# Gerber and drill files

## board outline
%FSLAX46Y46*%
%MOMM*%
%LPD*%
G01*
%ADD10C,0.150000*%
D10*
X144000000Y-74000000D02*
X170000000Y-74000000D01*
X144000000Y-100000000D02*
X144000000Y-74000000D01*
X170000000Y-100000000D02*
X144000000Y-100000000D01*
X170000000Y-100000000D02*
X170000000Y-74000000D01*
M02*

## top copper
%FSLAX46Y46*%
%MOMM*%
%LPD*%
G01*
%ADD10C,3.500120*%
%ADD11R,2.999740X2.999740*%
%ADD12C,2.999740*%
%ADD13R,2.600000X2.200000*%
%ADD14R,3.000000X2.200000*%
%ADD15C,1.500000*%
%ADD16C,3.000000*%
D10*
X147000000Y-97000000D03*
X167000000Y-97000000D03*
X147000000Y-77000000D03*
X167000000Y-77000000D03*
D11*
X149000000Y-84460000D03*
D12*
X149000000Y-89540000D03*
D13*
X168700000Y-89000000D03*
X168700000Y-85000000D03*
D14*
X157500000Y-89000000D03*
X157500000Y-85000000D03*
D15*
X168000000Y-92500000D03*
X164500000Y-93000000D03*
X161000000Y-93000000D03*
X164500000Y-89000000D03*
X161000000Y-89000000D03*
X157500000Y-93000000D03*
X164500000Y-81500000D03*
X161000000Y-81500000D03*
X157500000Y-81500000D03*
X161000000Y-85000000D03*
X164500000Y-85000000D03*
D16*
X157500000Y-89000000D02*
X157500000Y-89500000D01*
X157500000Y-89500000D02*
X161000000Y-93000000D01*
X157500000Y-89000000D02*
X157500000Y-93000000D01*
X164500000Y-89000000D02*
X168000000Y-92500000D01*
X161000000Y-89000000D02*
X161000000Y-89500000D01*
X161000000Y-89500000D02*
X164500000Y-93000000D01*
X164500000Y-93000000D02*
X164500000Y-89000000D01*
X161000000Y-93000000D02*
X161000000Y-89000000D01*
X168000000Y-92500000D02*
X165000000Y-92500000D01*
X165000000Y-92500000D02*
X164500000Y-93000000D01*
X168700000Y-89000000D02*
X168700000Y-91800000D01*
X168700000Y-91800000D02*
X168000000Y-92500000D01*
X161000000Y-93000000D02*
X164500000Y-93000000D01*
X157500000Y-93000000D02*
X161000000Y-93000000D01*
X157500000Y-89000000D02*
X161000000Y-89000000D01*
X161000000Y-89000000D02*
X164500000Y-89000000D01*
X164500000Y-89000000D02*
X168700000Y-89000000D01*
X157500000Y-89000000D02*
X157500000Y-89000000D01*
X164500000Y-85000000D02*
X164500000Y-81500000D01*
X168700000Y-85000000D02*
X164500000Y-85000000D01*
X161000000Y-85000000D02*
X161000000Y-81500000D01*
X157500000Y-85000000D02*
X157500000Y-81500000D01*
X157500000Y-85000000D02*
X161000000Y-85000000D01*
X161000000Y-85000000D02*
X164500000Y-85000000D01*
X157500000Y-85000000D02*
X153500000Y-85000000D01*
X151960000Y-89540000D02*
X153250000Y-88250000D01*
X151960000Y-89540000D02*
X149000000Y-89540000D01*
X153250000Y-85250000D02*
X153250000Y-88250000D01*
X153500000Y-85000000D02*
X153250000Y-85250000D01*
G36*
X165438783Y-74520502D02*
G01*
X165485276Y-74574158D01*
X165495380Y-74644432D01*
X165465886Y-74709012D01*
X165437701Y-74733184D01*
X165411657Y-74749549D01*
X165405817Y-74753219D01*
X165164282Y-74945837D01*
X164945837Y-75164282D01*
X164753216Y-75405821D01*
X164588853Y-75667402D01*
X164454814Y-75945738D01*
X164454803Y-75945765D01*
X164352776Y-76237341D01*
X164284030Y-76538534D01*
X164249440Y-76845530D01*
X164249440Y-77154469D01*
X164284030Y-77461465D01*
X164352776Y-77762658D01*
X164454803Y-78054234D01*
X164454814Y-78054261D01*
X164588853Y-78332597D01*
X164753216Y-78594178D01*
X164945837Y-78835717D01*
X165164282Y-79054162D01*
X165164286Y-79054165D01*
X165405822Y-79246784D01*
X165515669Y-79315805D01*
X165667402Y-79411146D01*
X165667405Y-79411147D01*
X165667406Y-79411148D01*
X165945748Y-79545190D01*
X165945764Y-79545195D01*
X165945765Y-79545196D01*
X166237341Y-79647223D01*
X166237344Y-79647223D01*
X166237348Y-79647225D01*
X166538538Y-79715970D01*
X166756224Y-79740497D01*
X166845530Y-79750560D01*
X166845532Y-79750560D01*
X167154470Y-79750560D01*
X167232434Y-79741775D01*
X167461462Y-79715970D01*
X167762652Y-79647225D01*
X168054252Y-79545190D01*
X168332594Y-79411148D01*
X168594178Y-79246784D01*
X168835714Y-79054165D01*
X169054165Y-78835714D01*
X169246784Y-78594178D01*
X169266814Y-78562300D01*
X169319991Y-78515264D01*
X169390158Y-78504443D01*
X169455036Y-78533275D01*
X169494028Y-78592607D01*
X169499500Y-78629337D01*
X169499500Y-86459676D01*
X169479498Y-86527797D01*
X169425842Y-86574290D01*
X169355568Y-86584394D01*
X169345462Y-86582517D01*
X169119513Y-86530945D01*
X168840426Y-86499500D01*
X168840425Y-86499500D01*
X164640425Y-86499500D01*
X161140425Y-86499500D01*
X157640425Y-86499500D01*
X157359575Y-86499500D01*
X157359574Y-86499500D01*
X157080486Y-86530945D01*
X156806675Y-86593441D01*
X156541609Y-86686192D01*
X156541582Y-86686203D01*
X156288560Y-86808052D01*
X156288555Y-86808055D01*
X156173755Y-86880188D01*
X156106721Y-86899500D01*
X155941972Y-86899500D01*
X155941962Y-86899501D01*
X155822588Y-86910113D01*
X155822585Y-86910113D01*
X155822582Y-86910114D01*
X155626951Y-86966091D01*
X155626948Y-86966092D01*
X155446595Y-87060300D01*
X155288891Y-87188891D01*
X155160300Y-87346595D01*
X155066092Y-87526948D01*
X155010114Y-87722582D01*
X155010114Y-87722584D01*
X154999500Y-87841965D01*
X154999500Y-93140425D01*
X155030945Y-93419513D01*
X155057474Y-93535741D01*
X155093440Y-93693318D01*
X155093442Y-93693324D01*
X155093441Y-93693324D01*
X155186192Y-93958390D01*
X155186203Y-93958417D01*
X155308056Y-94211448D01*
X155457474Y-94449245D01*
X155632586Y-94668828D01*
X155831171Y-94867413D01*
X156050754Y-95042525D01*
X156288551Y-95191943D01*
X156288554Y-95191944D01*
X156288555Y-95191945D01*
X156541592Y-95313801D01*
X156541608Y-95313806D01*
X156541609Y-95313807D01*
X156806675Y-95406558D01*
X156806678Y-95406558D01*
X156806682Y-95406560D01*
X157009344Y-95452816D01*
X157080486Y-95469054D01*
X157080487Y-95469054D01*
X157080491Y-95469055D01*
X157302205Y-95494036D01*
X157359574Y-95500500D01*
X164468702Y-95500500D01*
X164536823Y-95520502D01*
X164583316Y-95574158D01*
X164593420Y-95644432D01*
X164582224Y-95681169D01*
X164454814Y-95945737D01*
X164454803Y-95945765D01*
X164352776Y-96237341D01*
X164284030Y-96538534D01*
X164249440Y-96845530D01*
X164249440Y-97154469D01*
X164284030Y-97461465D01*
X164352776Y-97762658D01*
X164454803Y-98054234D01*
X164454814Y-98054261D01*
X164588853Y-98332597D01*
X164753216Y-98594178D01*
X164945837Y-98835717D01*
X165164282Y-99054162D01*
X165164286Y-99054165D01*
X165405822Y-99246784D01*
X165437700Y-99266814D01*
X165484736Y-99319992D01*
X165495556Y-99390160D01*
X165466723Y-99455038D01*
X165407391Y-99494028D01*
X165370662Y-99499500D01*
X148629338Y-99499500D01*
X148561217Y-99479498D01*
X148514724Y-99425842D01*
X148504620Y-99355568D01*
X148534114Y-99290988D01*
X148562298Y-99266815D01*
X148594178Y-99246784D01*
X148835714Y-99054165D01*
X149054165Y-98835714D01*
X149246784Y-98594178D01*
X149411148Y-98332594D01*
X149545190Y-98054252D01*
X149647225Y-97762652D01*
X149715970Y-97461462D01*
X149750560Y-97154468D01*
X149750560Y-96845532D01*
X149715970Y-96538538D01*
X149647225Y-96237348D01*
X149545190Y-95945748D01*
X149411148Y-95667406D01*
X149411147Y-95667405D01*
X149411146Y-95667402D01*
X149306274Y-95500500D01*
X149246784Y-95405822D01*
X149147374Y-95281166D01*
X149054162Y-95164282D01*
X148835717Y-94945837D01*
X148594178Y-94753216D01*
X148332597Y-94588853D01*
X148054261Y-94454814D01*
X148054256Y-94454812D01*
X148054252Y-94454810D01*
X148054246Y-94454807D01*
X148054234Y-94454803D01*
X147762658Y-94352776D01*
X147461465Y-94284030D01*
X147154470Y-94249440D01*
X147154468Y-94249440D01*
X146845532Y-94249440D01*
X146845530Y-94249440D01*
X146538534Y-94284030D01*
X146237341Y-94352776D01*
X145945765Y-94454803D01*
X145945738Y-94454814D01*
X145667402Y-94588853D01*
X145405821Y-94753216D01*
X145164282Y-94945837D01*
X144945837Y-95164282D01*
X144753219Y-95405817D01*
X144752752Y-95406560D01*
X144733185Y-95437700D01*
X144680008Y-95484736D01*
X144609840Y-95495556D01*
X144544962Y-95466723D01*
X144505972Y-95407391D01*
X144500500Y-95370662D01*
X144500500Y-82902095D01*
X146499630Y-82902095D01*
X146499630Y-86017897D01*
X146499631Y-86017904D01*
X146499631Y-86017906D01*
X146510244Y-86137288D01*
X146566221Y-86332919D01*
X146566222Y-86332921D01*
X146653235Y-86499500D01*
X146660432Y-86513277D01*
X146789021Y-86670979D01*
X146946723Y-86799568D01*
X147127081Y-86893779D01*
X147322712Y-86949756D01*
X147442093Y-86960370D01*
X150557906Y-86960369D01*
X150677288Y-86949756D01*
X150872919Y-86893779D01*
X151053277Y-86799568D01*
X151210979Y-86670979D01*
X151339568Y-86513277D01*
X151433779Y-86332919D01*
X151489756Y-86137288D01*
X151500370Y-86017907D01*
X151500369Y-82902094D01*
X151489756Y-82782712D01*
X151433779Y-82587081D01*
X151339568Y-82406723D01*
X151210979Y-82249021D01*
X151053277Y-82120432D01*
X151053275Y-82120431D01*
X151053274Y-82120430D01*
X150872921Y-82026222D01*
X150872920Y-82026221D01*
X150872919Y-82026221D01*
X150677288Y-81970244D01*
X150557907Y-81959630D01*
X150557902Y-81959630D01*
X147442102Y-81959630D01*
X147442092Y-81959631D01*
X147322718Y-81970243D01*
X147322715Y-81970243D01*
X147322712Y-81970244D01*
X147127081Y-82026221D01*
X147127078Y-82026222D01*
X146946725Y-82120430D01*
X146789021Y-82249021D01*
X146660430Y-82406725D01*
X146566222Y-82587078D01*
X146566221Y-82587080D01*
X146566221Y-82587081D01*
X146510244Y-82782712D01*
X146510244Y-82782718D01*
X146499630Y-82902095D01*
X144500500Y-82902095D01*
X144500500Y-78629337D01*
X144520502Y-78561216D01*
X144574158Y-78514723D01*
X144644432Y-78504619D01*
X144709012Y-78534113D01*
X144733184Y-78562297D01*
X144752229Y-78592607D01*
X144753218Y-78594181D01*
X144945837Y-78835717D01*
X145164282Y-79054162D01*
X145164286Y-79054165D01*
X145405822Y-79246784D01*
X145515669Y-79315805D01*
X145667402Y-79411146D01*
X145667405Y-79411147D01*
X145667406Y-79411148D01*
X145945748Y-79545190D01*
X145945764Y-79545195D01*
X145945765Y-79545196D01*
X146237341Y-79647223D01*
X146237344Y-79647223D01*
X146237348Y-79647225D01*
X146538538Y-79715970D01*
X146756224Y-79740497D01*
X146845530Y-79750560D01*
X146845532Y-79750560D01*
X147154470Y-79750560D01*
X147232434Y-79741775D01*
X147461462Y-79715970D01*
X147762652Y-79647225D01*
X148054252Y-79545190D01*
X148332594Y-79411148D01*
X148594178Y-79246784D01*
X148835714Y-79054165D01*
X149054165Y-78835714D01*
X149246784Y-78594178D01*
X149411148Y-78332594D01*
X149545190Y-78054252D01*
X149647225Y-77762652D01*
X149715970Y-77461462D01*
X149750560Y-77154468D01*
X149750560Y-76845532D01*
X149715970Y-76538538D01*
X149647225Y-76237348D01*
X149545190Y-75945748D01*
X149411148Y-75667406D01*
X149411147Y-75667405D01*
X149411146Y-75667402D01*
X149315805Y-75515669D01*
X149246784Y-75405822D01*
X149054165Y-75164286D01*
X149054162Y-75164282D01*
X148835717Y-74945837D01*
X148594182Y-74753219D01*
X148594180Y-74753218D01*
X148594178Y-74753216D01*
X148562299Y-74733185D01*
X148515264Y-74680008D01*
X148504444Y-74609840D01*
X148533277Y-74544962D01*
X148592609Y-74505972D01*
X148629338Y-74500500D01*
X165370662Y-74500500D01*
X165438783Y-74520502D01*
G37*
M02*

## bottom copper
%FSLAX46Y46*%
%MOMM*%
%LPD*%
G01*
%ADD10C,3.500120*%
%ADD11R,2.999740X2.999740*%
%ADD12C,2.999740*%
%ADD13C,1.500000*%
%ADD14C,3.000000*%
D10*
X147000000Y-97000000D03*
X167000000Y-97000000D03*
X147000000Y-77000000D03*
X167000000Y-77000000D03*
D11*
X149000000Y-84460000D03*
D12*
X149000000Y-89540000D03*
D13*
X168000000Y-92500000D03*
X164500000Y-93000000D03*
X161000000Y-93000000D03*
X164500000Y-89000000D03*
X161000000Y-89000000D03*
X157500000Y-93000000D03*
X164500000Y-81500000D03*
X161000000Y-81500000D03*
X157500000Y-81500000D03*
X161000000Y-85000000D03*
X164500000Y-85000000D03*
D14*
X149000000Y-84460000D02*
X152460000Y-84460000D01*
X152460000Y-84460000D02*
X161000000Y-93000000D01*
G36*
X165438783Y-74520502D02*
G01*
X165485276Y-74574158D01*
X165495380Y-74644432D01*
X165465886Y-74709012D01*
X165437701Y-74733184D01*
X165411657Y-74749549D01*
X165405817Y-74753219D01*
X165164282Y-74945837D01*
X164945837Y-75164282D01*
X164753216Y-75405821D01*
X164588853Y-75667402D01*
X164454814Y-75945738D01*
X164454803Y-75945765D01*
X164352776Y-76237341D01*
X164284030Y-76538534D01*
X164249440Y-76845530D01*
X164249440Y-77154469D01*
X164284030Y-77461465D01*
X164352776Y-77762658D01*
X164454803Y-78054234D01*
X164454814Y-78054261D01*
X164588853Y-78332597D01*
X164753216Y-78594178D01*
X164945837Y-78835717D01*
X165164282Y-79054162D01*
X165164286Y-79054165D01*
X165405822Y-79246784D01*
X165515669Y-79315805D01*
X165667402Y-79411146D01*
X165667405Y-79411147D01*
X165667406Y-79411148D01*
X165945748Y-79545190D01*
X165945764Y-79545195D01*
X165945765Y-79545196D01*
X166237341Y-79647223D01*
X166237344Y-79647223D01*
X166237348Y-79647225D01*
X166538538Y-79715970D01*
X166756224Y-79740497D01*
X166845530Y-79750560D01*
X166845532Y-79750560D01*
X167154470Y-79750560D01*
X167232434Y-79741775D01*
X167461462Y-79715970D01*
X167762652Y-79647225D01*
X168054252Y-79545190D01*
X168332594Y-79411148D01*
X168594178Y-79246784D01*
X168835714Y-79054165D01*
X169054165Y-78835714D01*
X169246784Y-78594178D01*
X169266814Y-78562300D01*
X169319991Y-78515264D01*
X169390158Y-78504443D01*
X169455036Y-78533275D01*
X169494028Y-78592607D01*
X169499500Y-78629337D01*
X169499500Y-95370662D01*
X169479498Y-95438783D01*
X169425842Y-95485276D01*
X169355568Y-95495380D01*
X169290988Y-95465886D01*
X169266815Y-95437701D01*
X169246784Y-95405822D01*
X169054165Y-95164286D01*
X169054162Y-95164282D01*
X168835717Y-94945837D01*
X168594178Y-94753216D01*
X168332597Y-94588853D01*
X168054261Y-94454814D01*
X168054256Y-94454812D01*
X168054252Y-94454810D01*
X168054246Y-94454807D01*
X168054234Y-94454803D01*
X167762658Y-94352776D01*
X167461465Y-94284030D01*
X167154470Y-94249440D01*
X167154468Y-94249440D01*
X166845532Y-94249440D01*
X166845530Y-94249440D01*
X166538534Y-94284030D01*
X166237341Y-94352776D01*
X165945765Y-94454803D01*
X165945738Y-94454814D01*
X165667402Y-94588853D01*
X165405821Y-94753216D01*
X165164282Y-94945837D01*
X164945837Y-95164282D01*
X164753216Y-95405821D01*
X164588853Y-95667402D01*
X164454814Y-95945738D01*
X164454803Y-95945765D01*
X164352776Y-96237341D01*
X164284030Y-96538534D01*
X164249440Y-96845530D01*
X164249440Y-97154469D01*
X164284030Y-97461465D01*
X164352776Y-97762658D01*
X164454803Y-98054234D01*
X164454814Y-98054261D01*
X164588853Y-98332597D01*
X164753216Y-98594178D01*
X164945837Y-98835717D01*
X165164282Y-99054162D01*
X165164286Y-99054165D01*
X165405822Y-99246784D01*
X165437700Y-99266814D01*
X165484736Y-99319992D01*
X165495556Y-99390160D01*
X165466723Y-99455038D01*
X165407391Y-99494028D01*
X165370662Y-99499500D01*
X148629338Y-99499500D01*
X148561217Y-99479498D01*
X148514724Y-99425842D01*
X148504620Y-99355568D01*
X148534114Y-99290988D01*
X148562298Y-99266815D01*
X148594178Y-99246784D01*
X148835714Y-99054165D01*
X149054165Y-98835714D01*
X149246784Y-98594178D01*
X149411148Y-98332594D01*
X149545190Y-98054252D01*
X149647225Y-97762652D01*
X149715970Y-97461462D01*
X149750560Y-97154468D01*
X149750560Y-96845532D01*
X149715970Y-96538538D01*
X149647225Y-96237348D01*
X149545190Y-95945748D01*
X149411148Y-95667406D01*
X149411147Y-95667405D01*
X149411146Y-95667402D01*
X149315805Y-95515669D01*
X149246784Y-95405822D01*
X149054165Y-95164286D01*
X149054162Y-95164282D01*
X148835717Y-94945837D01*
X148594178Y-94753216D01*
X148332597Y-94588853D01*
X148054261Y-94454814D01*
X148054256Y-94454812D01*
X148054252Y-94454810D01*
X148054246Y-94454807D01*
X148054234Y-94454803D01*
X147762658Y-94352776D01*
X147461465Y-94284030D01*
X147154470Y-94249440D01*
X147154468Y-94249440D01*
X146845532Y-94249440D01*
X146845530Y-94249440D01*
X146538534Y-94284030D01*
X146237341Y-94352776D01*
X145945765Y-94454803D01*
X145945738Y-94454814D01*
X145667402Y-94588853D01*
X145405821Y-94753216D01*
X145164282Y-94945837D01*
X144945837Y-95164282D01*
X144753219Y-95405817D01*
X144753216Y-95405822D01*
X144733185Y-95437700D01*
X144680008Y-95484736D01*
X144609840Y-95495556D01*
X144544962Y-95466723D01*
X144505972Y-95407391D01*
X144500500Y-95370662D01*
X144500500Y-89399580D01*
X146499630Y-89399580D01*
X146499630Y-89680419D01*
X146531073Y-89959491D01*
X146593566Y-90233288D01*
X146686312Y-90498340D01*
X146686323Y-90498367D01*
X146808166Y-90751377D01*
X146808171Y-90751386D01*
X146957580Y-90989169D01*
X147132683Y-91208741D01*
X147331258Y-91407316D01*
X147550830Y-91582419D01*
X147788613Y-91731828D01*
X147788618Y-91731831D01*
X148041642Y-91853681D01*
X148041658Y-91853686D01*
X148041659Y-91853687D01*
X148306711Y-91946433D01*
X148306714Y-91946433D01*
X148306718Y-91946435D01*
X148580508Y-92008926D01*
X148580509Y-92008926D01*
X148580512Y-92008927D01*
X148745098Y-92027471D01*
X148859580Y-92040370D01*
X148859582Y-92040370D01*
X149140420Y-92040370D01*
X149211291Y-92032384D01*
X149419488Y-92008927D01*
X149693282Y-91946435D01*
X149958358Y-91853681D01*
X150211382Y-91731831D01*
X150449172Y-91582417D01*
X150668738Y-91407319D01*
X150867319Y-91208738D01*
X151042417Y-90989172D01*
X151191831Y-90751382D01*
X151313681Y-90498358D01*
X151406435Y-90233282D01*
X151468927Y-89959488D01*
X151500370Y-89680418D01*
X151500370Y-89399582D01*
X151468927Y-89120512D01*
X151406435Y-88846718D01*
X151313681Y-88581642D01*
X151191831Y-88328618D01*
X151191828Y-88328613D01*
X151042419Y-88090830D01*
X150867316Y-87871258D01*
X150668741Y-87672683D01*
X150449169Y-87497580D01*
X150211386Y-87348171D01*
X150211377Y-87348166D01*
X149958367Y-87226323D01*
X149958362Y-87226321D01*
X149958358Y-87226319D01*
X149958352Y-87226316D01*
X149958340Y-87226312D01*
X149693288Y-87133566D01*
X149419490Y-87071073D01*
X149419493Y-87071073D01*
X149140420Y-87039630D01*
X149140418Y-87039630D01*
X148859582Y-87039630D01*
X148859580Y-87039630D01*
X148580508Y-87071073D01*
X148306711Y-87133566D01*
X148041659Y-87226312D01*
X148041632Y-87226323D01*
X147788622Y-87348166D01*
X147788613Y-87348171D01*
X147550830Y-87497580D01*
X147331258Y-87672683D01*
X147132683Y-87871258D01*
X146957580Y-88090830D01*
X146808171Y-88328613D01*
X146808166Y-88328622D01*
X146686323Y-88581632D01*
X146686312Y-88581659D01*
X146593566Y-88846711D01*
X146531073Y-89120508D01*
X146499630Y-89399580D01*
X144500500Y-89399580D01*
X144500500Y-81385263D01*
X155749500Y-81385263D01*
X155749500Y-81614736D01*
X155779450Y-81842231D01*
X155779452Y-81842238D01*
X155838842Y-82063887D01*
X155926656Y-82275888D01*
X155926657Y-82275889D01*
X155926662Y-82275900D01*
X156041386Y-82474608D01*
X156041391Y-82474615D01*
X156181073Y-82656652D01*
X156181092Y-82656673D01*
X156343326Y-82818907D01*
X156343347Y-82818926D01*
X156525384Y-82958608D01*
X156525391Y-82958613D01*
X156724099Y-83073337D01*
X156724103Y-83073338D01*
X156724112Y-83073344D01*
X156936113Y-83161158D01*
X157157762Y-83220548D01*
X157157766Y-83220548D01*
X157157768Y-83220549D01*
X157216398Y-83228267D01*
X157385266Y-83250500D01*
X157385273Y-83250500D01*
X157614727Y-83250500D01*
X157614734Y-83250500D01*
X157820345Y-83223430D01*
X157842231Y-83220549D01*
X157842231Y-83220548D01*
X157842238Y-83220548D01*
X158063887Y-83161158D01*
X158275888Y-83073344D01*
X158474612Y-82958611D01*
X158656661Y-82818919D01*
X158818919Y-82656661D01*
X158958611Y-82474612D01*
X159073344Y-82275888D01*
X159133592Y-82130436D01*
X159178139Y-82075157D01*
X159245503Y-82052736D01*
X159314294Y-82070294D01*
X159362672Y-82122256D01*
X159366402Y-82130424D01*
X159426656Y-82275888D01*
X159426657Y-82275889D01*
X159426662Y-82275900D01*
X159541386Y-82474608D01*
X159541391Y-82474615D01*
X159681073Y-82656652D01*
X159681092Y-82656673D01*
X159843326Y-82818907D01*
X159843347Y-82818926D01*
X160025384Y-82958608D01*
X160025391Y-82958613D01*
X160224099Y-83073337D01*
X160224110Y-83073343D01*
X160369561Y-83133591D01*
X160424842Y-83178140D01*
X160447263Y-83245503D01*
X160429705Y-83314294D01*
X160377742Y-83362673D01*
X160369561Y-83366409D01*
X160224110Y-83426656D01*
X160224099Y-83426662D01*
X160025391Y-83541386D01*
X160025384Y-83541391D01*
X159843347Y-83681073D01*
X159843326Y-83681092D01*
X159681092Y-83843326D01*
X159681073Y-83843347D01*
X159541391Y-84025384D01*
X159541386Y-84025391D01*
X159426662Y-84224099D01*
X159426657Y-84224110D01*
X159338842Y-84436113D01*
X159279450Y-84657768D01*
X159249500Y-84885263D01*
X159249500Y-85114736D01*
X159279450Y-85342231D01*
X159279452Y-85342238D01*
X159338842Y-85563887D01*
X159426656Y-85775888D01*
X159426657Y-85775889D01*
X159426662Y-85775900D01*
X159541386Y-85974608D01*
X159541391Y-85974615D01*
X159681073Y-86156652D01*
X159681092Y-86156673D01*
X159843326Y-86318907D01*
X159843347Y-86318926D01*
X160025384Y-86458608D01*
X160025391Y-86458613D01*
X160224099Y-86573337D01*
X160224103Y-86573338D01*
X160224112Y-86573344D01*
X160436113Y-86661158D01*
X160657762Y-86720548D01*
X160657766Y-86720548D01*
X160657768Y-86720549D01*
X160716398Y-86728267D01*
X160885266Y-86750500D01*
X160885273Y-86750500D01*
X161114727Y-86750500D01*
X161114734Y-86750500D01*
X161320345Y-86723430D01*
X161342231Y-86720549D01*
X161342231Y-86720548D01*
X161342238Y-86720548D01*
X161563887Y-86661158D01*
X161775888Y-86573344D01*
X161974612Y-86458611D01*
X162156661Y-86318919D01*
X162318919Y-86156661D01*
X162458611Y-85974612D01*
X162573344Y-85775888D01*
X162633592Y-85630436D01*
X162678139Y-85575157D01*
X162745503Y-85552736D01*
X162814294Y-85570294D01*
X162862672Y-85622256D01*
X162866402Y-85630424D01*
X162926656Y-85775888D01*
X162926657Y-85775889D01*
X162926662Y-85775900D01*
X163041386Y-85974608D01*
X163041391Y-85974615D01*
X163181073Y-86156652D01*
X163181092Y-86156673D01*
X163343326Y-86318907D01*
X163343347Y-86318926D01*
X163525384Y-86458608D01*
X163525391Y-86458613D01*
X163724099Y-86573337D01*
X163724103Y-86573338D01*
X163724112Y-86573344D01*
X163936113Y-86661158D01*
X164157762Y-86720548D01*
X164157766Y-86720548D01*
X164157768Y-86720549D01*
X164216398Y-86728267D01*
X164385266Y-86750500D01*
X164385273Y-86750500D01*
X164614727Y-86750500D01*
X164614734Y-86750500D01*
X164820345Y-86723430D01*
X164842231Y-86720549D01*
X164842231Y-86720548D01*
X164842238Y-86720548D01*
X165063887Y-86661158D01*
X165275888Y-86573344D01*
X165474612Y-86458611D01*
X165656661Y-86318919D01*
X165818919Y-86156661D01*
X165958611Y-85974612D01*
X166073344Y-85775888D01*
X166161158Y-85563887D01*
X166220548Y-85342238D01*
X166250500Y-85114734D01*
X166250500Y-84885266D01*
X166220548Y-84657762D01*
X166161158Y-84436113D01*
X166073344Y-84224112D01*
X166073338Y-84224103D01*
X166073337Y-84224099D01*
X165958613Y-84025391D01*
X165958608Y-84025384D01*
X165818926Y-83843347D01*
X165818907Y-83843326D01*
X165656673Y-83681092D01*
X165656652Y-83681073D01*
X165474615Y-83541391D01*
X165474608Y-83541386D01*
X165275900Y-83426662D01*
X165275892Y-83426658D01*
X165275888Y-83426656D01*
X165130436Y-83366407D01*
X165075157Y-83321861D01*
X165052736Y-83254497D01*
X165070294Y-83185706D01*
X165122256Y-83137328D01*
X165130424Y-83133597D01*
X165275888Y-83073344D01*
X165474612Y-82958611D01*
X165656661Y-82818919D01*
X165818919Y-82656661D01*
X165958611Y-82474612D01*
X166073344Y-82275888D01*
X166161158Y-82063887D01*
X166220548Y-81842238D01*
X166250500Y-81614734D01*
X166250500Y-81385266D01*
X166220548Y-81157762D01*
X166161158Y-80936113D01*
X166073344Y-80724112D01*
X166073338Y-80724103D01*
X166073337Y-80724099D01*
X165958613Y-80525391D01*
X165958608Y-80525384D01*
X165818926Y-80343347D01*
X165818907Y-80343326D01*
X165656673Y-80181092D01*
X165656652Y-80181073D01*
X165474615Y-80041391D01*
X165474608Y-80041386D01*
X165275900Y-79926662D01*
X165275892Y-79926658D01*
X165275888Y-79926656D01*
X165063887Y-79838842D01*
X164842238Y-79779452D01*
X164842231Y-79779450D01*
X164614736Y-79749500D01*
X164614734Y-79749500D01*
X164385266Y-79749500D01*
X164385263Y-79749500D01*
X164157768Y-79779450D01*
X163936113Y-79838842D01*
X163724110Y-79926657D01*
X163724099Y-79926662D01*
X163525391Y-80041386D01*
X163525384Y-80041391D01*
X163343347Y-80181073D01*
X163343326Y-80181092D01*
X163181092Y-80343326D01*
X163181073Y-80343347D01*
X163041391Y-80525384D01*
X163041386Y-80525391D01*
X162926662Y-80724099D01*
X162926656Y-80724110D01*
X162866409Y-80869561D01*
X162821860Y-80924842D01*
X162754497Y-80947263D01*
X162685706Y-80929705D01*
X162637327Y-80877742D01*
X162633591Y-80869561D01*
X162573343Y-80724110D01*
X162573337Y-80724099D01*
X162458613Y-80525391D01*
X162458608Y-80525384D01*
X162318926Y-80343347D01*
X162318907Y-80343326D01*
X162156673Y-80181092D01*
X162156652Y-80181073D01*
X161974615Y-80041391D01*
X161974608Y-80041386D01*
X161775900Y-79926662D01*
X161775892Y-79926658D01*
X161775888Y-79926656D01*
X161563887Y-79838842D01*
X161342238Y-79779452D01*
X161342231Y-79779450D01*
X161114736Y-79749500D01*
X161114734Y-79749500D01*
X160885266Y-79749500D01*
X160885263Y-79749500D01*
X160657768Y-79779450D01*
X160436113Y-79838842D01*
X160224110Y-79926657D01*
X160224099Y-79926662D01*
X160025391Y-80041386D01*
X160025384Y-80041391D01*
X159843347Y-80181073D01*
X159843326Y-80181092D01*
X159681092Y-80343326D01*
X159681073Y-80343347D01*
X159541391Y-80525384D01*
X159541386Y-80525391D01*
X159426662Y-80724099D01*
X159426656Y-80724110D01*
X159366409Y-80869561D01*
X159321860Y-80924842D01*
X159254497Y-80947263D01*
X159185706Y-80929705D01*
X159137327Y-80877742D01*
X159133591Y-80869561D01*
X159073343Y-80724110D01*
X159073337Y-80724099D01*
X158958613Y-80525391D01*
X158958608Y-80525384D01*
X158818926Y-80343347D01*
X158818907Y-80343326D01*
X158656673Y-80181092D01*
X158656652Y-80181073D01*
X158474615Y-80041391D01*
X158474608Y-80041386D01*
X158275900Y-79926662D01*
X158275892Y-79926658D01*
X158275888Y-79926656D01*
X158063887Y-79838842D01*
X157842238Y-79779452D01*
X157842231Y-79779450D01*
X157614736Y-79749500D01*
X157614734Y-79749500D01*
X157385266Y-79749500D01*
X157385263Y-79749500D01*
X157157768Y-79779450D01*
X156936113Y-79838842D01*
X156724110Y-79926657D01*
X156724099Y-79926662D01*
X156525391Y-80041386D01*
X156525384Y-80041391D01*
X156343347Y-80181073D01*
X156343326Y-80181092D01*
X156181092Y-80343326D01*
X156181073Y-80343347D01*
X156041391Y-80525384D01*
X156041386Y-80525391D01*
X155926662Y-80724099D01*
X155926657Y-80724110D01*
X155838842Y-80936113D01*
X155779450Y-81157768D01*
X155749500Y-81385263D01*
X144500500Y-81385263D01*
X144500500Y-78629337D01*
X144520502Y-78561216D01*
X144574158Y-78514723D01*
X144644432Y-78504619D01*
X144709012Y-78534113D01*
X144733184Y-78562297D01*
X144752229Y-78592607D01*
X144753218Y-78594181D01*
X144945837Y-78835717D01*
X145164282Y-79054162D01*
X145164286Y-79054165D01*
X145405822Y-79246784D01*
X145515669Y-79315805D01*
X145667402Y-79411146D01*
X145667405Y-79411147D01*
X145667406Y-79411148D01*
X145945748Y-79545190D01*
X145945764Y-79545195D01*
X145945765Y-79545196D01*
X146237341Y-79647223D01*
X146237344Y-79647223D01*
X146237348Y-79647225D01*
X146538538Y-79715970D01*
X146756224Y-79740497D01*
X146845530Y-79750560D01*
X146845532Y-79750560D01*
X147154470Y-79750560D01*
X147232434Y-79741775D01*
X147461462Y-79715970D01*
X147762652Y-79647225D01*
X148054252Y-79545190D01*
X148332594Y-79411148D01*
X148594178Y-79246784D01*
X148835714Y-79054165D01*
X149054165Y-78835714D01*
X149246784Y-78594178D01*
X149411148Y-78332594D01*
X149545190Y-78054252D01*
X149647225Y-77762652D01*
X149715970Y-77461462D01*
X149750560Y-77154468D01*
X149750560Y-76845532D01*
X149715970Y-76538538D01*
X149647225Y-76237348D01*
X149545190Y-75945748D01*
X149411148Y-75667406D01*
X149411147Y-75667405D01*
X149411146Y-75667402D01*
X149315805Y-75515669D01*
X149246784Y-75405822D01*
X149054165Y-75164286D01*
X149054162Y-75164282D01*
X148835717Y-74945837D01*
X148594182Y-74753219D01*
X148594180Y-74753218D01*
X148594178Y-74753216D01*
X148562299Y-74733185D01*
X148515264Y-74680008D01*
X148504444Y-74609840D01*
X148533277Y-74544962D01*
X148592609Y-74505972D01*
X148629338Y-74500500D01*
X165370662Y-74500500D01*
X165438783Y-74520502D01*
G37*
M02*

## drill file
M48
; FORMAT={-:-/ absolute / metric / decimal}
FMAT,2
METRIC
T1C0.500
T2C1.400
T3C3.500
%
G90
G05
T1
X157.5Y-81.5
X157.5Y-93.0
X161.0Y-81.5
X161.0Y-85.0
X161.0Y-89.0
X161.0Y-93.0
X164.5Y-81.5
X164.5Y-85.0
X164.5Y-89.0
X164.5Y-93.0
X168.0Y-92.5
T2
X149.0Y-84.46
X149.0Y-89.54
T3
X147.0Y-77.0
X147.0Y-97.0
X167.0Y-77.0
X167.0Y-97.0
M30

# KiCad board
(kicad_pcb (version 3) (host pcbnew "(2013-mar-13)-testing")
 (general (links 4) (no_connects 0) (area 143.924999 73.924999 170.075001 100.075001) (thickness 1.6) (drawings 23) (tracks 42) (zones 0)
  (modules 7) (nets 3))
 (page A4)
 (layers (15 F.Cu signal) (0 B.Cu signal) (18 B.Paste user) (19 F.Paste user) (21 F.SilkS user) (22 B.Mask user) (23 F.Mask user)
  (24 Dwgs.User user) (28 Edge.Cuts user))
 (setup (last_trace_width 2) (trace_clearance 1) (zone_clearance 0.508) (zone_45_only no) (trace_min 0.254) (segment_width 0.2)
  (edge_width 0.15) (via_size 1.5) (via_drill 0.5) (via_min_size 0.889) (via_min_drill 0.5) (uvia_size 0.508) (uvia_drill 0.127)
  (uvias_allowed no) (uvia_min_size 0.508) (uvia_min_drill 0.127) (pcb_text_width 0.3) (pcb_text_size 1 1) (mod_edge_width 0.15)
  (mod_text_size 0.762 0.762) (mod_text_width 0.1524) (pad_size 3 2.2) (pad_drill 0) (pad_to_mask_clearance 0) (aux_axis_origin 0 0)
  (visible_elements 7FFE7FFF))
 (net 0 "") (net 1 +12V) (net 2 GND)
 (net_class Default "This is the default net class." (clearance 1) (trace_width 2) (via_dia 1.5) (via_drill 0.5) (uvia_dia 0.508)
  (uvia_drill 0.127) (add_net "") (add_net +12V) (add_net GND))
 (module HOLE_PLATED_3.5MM (layer F.Cu) (at 147 97)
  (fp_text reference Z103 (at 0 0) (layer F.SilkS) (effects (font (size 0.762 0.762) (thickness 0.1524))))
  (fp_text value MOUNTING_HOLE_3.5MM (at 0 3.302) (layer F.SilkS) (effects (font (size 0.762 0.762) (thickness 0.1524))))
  (pad 1 thru_hole circle (at 0 0) (size 3.50012 3.50012) (drill 3.500119) (layers *.Cu F.SilkS)))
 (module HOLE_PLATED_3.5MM (layer F.Cu) (at 167 97)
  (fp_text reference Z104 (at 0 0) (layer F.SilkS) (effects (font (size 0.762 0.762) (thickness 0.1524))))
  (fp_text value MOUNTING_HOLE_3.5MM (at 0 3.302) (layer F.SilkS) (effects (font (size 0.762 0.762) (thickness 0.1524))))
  (pad 1 thru_hole circle (at 0 0) (size 3.50012 3.50012) (drill 3.500119) (layers *.Cu F.SilkS)))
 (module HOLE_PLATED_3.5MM (layer F.Cu) (at 147 77)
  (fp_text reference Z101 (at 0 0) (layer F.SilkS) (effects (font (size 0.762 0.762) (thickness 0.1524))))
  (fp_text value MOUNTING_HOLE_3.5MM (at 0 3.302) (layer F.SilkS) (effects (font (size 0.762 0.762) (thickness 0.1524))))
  (pad 1 thru_hole circle (at 0 0) (size 3.50012 3.50012) (drill 3.500119) (layers *.Cu F.SilkS)))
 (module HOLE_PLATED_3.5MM (layer F.Cu) (at 167 77)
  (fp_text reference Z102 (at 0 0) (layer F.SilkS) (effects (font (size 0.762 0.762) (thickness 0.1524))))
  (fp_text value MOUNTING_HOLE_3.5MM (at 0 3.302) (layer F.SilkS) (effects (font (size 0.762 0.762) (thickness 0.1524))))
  (pad 1 thru_hole circle (at 0 0) (size 3.50012 3.50012) (drill 3.500119) (layers *.Cu F.SilkS)))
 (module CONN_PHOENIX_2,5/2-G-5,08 (layer F.Cu) (at 149 87 270)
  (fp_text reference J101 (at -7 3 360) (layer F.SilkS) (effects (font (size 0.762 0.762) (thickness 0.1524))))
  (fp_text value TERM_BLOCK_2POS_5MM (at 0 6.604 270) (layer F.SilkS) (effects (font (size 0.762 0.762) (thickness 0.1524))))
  (pad 1 thru_hole rect (at -2.54 0 270) (size 2.99974 2.99974) (drill 1.39954) (layers *.Cu *.Mask F.SilkS) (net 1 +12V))
  (pad 2 thru_hole circle (at 2.54 0 270) (size 2.99974 2.99974) (drill 1.39954) (layers *.Cu *.Mask F.SilkS) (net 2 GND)))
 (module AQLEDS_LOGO (layer F.Cu) (at 157 97)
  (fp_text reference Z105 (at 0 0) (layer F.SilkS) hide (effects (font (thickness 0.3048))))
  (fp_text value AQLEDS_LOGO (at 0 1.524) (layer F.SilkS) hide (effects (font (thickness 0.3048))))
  (pad "" connect rect (at -2.24028 -1.69164) (size 0.82296 0.09144) (layers F.SilkS) (clearance 0.0254))
  (pad "" connect rect (at 0.50292 -1.69164) (size 0.64008 0.09144) (layers F.SilkS) (clearance 0.0254))
  (pad "" connect rect (at 1.69164 -1.69164) (size 1.00584 0.09144) (layers F.SilkS) (clearance 0.0254))
  (pad "" connect rect (at 2.78892 -1.69164) (size 1.00584 0.09144) (layers F.SilkS) (clearance 0.0254))
  (pad "" connect rect (at -2.286 -1.6002) (size 0.9144 0.09144) (layers F.SilkS) (clearance 0.0254))
  (pad "" connect rect (at 0.4572 -1.6002) (size 0.73152 0.09144) (layers F.SilkS) (clearance 0.0254))
  (pad "" connect rect (at 2.286 -1.6002) (size 2.19456 0.09144) (layers F.SilkS) (clearance 0.0254))
  (pad "" connect rect (at -2.33172 -1.50876) (size 0.82296 0.09144) (layers F.SilkS) (clearance 0.0254))
  (pad "" connect rect (at 0.4572 -1.50876) (size 0.73152 0.09144) (layers F.SilkS) (clearance 0.0254))
  (pad "" connect rect (at 2.286 -1.50876) (size 2.37744 0.09144) (layers F.SilkS) (clearance 0.0254))
  (pad "" connect rect (at -2.37744 -1.41732) (size 0.9144 0.09144) (layers F.SilkS) (clearance 0.0254))
  (pad "" connect rect (at 0.41148 -1.41732) (size 0.64008 0.09144) (layers F.SilkS) (clearance 0.0254))
  (pad "" connect rect (at 2.286 -1.41732) (size 2.37744 0.09144) (layers F.SilkS) (clearance 0.0254))
  (pad "" connect rect (at -2.42316 -1.32588) (size 1.00584 0.09144) (layers F.SilkS) (clearance 0.0254))
  (pad "" connect rect (at 0.41148 -1.32588) (size 0.64008 0.09144) (layers F.SilkS) (clearance 0.0254))
  (pad "" connect rect (at 2.286 -1.32588) (size 2.37744 0.09144) (layers F.SilkS) (clearance 0.0254))
  (pad "" connect rect (at -2.5146 -1.23444) (size 1.00584 0.09144) (layers F.SilkS) (clearance 0.0254))
  (pad "" connect rect (at 0.36576 -1.23444) (size 0.73152 0.09144) (layers F.SilkS) (clearance 0.0254))
  (pad "" connect rect (at 1.50876 -1.23444) (size 1.00584 0.09144) (layers F.SilkS) (clearance 0.0254))
  (pad "" connect rect (at 2.37744 -1.23444) (size 0.54864 0.09144) (layers F.SilkS) (clearance 0.0254))
  (pad "" connect rect (at 3.06324 -1.23444) (size 0.64008 0.09144) (layers F.SilkS) (clearance 0.0254))
  (pad "" connect rect (at -2.5146 -1.143) (size 1.00584 0.09144) (layers F.SilkS) (clearance 0.0254))
  (pad "" connect rect (at 0.32004 -1.143) (size 0.64008 0.09144) (layers F.SilkS) (clearance 0.0254))
  (pad "" connect rect (at 1.3716 -1.143) (size 0.73152 0.09144) (layers F.SilkS) (clearance 0.0254))
  (pad "" connect rect (at 2.37744 -1.143) (size 0.54864 0.09144) (layers F.SilkS) (clearance 0.0254))
  (pad "" connect rect (at 3.10896 -1.143) (size 0.54864 0.09144) (layers F.SilkS) (clearance 0.0254))
  (pad "" connect rect (at -2.56032 -1.05156) (size 1.09728 0.09144) (layers F.SilkS) (clearance 0.0254))
  (pad "" connect rect (at 0.32004 -1.05156) (size 0.64008 0.09144) (layers F.SilkS) (clearance 0.0254))
  (pad "" connect rect (at 1.32588 -1.05156) (size 0.64008 0.09144) (layers F.SilkS) (clearance 0.0254))
  (pad "" connect rect (at 2.33172 -1.05156) (size 0.64008 0.09144) (layers F.SilkS) (clearance 0.0254))
  (pad "" connect rect (at 3.06324 -1.05156) (size 0.64008 0.09144) (layers F.SilkS) (clearance 0.0254))
  (pad "" connect rect (at -2.60604 -0.96012) (size 1.18872 0.09144) (layers F.SilkS) (clearance 0.0254))
  (pad "" connect rect (at 0.27432 -0.96012) (size 0.73152 0.09144) (layers F.SilkS) (clearance 0.0254))
  (pad "" connect rect (at 1.32588 -0.96012) (size 0.64008 0.09144) (layers F.SilkS) (clearance 0.0254))
  (pad "" connect rect (at 2.286 -0.96012) (size 0.54864 0.09144) (layers F.SilkS) (clearance 0.0254))
  (pad "" connect rect (at 3.01752 -0.96012) (size 0.54864 0.09144) (layers F.SilkS) (clearance 0.0254))
  (pad "" connect rect (at -2.69748 -0.86868) (size 1.18872 0.09144) (layers F.SilkS) (clearance 0.0254))
  (pad "" connect rect (at 0.27432 -0.86868) (size 0.73152 0.09144) (layers F.SilkS) (clearance 0.0254))
  (pad "" connect rect (at 1.28016 -0.86868) (size 0.73152 0.09144) (layers F.SilkS) (clearance 0.0254))
  (pad "" connect rect (at 2.286 -0.86868) (size 0.54864 0.09144) (layers F.SilkS) (clearance 0.0254))
  (pad "" connect rect (at 3.01752 -0.86868) (size 0.54864 0.09144) (layers F.SilkS) (clearance 0.0254))
  (pad "" connect rect (at -2.69748 -0.77724) (size 1.18872 0.09144) (layers F.SilkS) (clearance 0.0254))
  (pad "" connect rect (at 0.2286 -0.77724) (size 0.64008 0.09144) (layers F.SilkS) (clearance 0.0254))
  (pad "" connect rect (at 1.28016 -0.77724) (size 0.73152 0.09144) (layers F.SilkS) (clearance 0.0254))
  (pad "" connect rect (at 2.24028 -0.77724) (size 0.64008 0.09144) (layers F.SilkS) (clearance 0.0254))
  (pad "" connect rect (at 2.9718 -0.77724) (size 0.64008 0.09144) (layers F.SilkS) (clearance 0.0254))
  (pad "" connect rect (at -2.7432 -0.6858) (size 1.28016 0.09144) (layers F.SilkS) (clearance 0.0254))
  (pad "" connect rect (at 0.2286 -0.6858) (size 0.64008 0.09144) (layers F.SilkS) (clearance 0.0254))
  (pad "" connect rect (at 1.23444 -0.6858) (size 0.64008 0.09144) (layers F.SilkS) (clearance 0.0254))
  (pad "" connect rect (at 2.19456 -0.6858) (size 0.54864 0.09144) (layers F.SilkS) (clearance 0.0254))
  (pad "" connect rect (at 2.92608 -0.6858) (size 0.54864 0.09144) (layers F.SilkS) (clearance 0.0254))
  (pad "" connect rect (at -2.83464 -0.59436) (size 1.28016 0.09144) (layers F.SilkS) (clearance 0.0254))
  (pad "" connect rect (at 0.18288 -0.59436) (size 0.73152 0.09144) (layers F.SilkS) (clearance 0.0254))
  (pad "" connect rect (at 1.3716 -0.59436) (size 0.9144 0.09144) (layers F.SilkS) (clearance 0.0254))
  (pad "" connect rect (at 2.19456 -0.59436) (size 0.54864 0.09144) (layers F.SilkS) (clearance 0.0254))
  (pad "" connect rect (at 2.92608 -0.59436) (size 0.54864 0.09144) (layers F.SilkS) (clearance 0.0254))
  (pad "" connect rect (at -3.15468 -0.50292) (size 0.64008 0.09144) (layers F.SilkS) (clearance 0.0254))
  (pad "" connect rect (at -2.46888 -0.50292) (size 0.54864 0.09144) (layers F.SilkS) (clearance 0.0254))
  (pad "" connect rect (at 0.13716 -0.50292) (size 0.64008 0.09144) (layers F.SilkS) (clearance 0.0254))
  (pad "" connect rect (at 1.64592 -0.50292) (size 1.64592 0.09144) (layers F.SilkS) (clearance 0.0254))
  (pad "" connect rect (at 2.92608 -0.50292) (size 0.54864 0.09144) (layers F.SilkS) (clearance 0.0254))
  (pad "" connect rect (at -3.24612 -0.41148) (size 0.64008 0.09144) (layers F.SilkS) (clearance 0.0254))
  (pad "" connect rect (at -2.46888 -0.41148) (size 0.54864 0.09144) (layers F.SilkS) (clearance 0.0254))
  (pad "" connect rect (at -1.143 -0.41148) (size 1.18872 0.09144) (layers F.SilkS) (clearance 0.0254))
  (pad "" connect rect (at 0.13716 -0.41148) (size 0.64008 0.09144) (layers F.SilkS) (clearance 0.0254))
  (pad "" connect rect (at 1.6002 -0.41148) (size 1.55448 0.09144) (layers F.SilkS) (clearance 0.0254))
  (pad "" connect rect (at 2.88036 -0.41148) (size 0.64008 0.09144) (layers F.SilkS) (clearance 0.0254))
  (pad "" connect rect (at 4.06908 -0.41148) (size 1.18872 0.09144) (layers F.SilkS) (clearance 0.0254))
  (pad "" connect rect (at -3.29184 -0.32004) (size 0.73152 0.09144) (layers F.SilkS) (clearance 0.0254))
  (pad "" connect rect (at -2.56032 -0.32004) (size 0.54864 0.09144) (layers F.SilkS) (clearance 0.0254))
  (pad "" connect rect (at -1.143 -0.32004) (size 1.55448 0.09144) (layers F.SilkS) (clearance 0.0254))
  (pad "" connect rect (at 0.09144 -0.32004) (size 0.73152 0.09144) (layers F.SilkS) (clearance 0.0254))
  (pad "" connect rect (at 1.6002 -0.32004) (size 1.55448 0.09144) (layers F.SilkS) (clearance 0.0254))
  (pad "" connect rect (at 2.83464 -0.32004) (size 0.54864 0.09144) (layers F.SilkS) (clearance 0.0254))
  (pad "" connect rect (at 4.02336 -0.32004) (size 1.28016 0.09144) (layers F.SilkS) (clearance 0.0254))
  (pad "" connect rect (at -3.38328 -0.2286) (size 0.73152 0.09144) (layers F.SilkS) (clearance 0.0254))
  (pad "" connect rect (at -2.56032 -0.2286) (size 0.54864 0.09144) (layers F.SilkS) (clearance 0.0254))
  (pad "" connect rect (at -0.77724 -0.2286) (size 2.46888 0.09144) (layers F.SilkS) (clearance 0.0254))
  (pad "" connect rect (at 1.55448 -0.2286) (size 1.64592 0.09144) (layers F.SilkS) (clearance 0.0254))
  (pad "" connect rect (at 2.83464 -0.2286) (size 0.54864 0.09144) (layers F.SilkS) (clearance 0.0254))
  (pad "" connect rect (at 3.97764 -0.2286) (size 1.3716 0.09144) (layers F.SilkS) (clearance 0.0254))
  (pad "" connect rect (at -3.38328 -0.13716) (size 0.73152 0.09144) (layers F.SilkS) (clearance 0.0254))
  (pad "" connect rect (at -2.56032 -0.13716) (size 0.54864 0.09144) (layers F.SilkS) (clearance 0.0254))
  (pad "" connect rect (at -0.86868 -0.13716) (size 2.46888 0.09144) (layers F.SilkS) (clearance 0.0254))
  (pad "" connect rect (at 1.55448 -0.13716) (size 1.64592 0.09144) (layers F.SilkS) (clearance 0.0254))
  (pad "" connect rect (at 2.83464 -0.13716) (size 0.54864 0.09144) (layers F.SilkS) (clearance 0.0254))
  (pad "" connect rect (at 3.93192 -0.13716) (size 1.46304 0.09144) (layers F.SilkS) (clearance 0.0254))
  (pad "" connect rect (at -3.47472 -0.04572) (size 0.73152 0.09144) (layers F.SilkS) (clearance 0.0254))
  (pad "" connect rect (at -2.56032 -0.04572) (size 0.54864 0.09144) (layers F.SilkS) (clearance 0.0254))
  (pad "" connect rect (at -0.9144 -0.04572) (size 2.56032 0.09144) (layers F.SilkS) (clearance 0.0254))
  (pad "" connect rect (at 1.18872 -0.04572) (size 0.9144 0.09144) (layers F.SilkS) (clearance 0.0254))
  (pad "" connect rect (at 2.01168 -0.04572) (size 0.54864 0.09144) (layers F.SilkS) (clearance 0.0254))
  (pad "" connect rect (at 2.7432 -0.04572) (size 0.54864 0.09144) (layers F.SilkS) (clearance 0.0254))
  (pad "" connect rect (at 3.8862 -0.04572) (size 1.55448 0.09144) (layers F.SilkS) (clearance 0.0254))
  (pad "" connect rect (at -3.56616 0.04572) (size 0.73152 0.09144) (layers F.SilkS) (clearance 0.0254))
  (pad "" connect rect (at -2.60604 0.04572) (size 0.4572 0.09144) (layers F.SilkS) (clearance 0.0254))
  (pad "" connect rect (at -0.9144 0.04572) (size 2.56032 0.09144) (layers F.SilkS) (clearance 0.0254))
  (pad "" connect rect (at 1.05156 0.04572) (size 0.64008 0.09144) (layers F.SilkS) (clearance 0.0254))
  (pad "" connect rect (at 2.01168 0.04572) (size 0.54864 0.09144) (layers F.SilkS) (clearance 0.0254))
  (pad "" connect rect (at 2.7432 0.04572) (size 0.54864 0.09144) (layers F.SilkS) (clearance 0.0254))
  (pad "" connect rect (at 3.52044 0.04572) (size 0.82296 0.09144) (layers F.SilkS) (clearance 0.0254))
  (pad "" connect rect (at -3.6576 0.13716) (size 0.73152 0.09144) (layers F.SilkS) (clearance 0.0254))
  (pad "" connect rect (at -2.65176 0.13716) (size 0.54864 0.09144) (layers F.SilkS) (clearance 0.0254))
  (pad "" connect rect (at -0.96012 0.13716) (size 2.46888 0.09144) (layers F.SilkS) (clearance 0.0254))
  (pad "" connect rect (at 1.00584 0.13716) (size 0.73152 0.09144) (layers F.SilkS) (clearance 0.0254))
  (pad "" connect rect (at 1.96596 0.13716) (size 0.64008 0.09144) (layers F.SilkS) (clearance 0.0254))
  (pad "" connect rect (at 2.7432 0.13716) (size 0.54864 0.09144) (layers F.SilkS) (clearance 0.0254))
  (pad "" connect rect (at 3.74904 0.13716) (size 1.28016 0.09144) (layers F.SilkS) (clearance 0.0254))
  (pad "" connect rect (at -3.52044 0.2286) (size 1.00584 0.09144) (layers F.SilkS) (clearance 0.0254))
  (pad "" connect rect (at -2.65176 0.2286) (size 0.54864 0.09144) (layers F.SilkS) (clearance 0.0254))
  (pad "" connect rect (at -1.87452 0.2286) (size 0.82296 0.09144) (layers F.SilkS) (clearance 0.0254))
  (pad "" connect rect (at -0.36576 0.2286) (size 1.28016 0.09144) (layers F.SilkS) (clearance 0.0254))
  (pad "" connect rect (at 0.96012 0.2286) (size 0.64008 0.09144) (layers F.SilkS) (clearance 0.0254))
  (pad "" connect rect (at 1.92024 0.2286) (size 0.54864 0.09144) (layers F.SilkS) (clearance 0.0254))
  (pad "" connect rect (at 2.65176 0.2286) (size 0.54864 0.09144) (layers F.SilkS) (clearance 0.0254))
  (pad "" connect rect (at 3.84048 0.2286) (size 1.28016 0.09144) (layers F.SilkS) (clearance 0.0254))
  (pad "" connect rect (at -3.29184 0.32004) (size 1.64592 0.09144) (layers F.SilkS) (clearance 0.0254))
  (pad "" connect rect (at -1.87452 0.32004) (size 0.82296 0.09144) (layers F.SilkS) (clearance 0.0254))
  (pad "" connect rect (at -0.41148 0.32004) (size 1.3716 0.09144) (layers F.SilkS) (clearance 0.0254))
  (pad "" connect rect (at 0.96012 0.32004) (size 0.64008 0.09144) (layers F.SilkS) (clearance 0.0254))
  (pad "" connect rect (at 1.92024 0.32004) (size 0.54864 0.09144) (layers F.SilkS) (clearance 0.0254))
  (pad "" connect rect (at 2.65176 0.32004) (size 0.54864 0.09144) (layers F.SilkS) (clearance 0.0254))
  (pad "" connect rect (at 3.84048 0.32004) (size 1.28016 0.09144) (layers F.SilkS) (clearance 0.0254))
  (pad "" connect rect (at -3.33756 0.41148) (size 1.73736 0.09144) (layers F.SilkS) (clearance 0.0254))
  (pad "" connect rect (at -1.87452 0.41148) (size 0.82296 0.09144) (layers F.SilkS) (clearance 0.0254))
  (pad "" connect rect (at -0.4572 0.41148) (size 1.28016 0.09144) (layers F.SilkS) (clearance 0.0254))
  (pad "" connect rect (at 0.9144 0.41148) (size 0.73152 0.09144) (layers F.SilkS) (clearance 0.0254))
  (pad "" connect rect (at 1.92024 0.41148) (size 0.54864 0.09144) (layers F.SilkS) (clearance 0.0254))
  (pad "" connect rect (at 2.65176 0.41148) (size 0.54864 0.09144) (layers F.SilkS) (clearance 0.0254))
  (pad "" connect rect (at 3.8862 0.41148) (size 1.18872 0.09144) (layers F.SilkS) (clearance 0.0254))
  (pad "" connect rect (at -3.38328 0.50292) (size 1.8288 0.09144) (layers F.SilkS) (clearance 0.0254))
  (pad "" connect rect (at -1.96596 0.50292) (size 0.82296 0.09144) (layers F.SilkS) (clearance 0.0254))
  (pad "" connect rect (at -0.32004 0.50292) (size 1.55448 0.09144) (layers F.SilkS) (clearance 0.0254))
  (pad "" connect rect (at 1.00584 0.50292) (size 0.9144 0.09144) (layers F.SilkS) (clearance 0.0254))
  (pad "" connect rect (at 1.8288 0.50292) (size 0.54864 0.09144) (layers F.SilkS) (clearance 0.0254))
  (pad "" connect rect (at 2.65176 0.50292) (size 0.54864 0.09144) (layers F.SilkS) (clearance 0.0254))
  (pad "" connect rect (at 3.93192 0.50292) (size 1.09728 0.09144) (layers F.SilkS) (clearance 0.0254))
  (pad "" connect rect (at -3.38328 0.59436) (size 1.8288 0.09144) (layers F.SilkS) (clearance 0.0254))
  (pad "" connect rect (at -1.96596 0.59436) (size 0.82296 0.09144) (layers F.SilkS) (clearance 0.0254))
  (pad "" connect rect (at 0.50292 0.59436) (size 3.2004 0.09144) (layers F.SilkS) (clearance 0.0254))
  (pad "" connect rect (at 2.56032 0.59436) (size 0.54864 0.09144) (layers F.SilkS) (clearance 0.0254))
  (pad "" connect rect (at 4.16052 0.59436) (size 0.64008 0.09144) (layers F.SilkS) (clearance 0.0254))
  (pad "" connect rect (at -3.47472 0.6858) (size 1.8288 0.09144) (layers F.SilkS) (clearance 0.0254))
  (pad "" connect rect (at -1.96596 0.6858) (size 0.82296 0.09144) (layers F.SilkS) (clearance 0.0254))
  (pad "" connect rect (at 0.82296 0.6858) (size 4.02336 0.09144) (layers F.SilkS) (clearance 0.0254))
  (pad "" connect rect (at 3.79476 0.6858) (size 1.3716 0.09144) (layers F.SilkS) (clearance 0.0254))
  (pad "" connect rect (at -4.06908 0.77724) (size 0.82296 0.09144) (layers F.SilkS) (clearance 0.0254))
  (pad "" connect rect (at -2.92608 0.77724) (size 0.73152 0.09144) (layers F.SilkS) (clearance 0.0254))
  (pad "" connect rect (at -1.96596 0.77724) (size 0.82296 0.09144) (layers F.SilkS) (clearance 0.0254))
  (pad "" connect rect (at 0.82296 0.77724) (size 4.02336 0.09144) (layers F.SilkS) (clearance 0.0254))
  (pad "" connect rect (at 3.74904 0.77724) (size 1.28016 0.09144) (layers F.SilkS) (clearance 0.0254))
  (pad "" connect rect (at -4.1148 0.86868) (size 0.73152 0.09144) (layers F.SilkS) (clearance 0.0254))
  (pad "" connect rect (at -2.92608 0.86868) (size 0.73152 0.09144) (layers F.SilkS) (clearance 0.0254))
  (pad "" connect rect (at -2.0574 0.86868) (size 0.82296 0.09144) (layers F.SilkS) (clearance 0.0254))
  (pad "" connect rect (at 0.77724 0.86868) (size 3.93192 0.09144) (layers F.SilkS) (clearance 0.0254))
  (pad "" connect rect (at 3.70332 0.86868) (size 1.3716 0.09144) (layers F.SilkS) (clearance 0.0254))
  (pad "" connect rect (at -4.16052 0.96012) (size 0.82296 0.09144) (layers F.SilkS) (clearance 0.0254))
  (pad "" connect rect (at -2.9718 0.96012) (size 0.64008 0.09144) (layers F.SilkS) (clearance 0.0254))
  (pad "" connect rect (at -2.0574 0.96012) (size 0.82296 0.09144) (layers F.SilkS) (clearance 0.0254))
  (pad "" connect rect (at 0.73152 0.96012) (size 4.02336 0.09144) (layers F.SilkS) (clearance 0.0254))
  (pad "" connect rect (at 3.6576 0.96012) (size 1.28016 0.09144) (layers F.SilkS) (clearance 0.0254))
  (pad "" connect rect (at -4.25196 1.05156) (size 0.82296 0.09144) (layers F.SilkS) (clearance 0.0254))
  (pad "" connect rect (at -2.9718 1.05156) (size 0.64008 0.09144) (layers F.SilkS) (clearance 0.0254))
  (pad "" connect rect (at -2.0574 1.05156) (size 0.82296 0.09144) (layers F.SilkS) (clearance 0.0254))
  (pad "" connect rect (at -0.50292 1.05156) (size 1.73736 0.09144) (layers F.SilkS) (clearance 0.0254))
  (pad "" connect rect (at 0.96012 1.05156) (size 1.00584 0.09144) (layers F.SilkS) (clearance 0.0254))
  (pad "" connect rect (at 2.0574 1.05156) (size 1.00584 0.09144) (layers F.SilkS) (clearance 0.0254))
  (pad "" connect rect (at 3.56616 1.05156) (size 1.09728 0.09144) (layers F.SilkS) (clearance 0.0254))
  (pad "" connect rect (at -4.3434 1.143) (size 0.82296 0.09144) (layers F.SilkS) (clearance 0.0254))
  (pad "" connect rect (at -1.50876 1.143) (size 1.92024 0.09144) (layers F.SilkS) (clearance 0.0254))
  (pad "" connect rect (at -4.38912 1.23444) (size 0.73152 0.09144) (layers F.SilkS) (clearance 0.0254))
  (pad "" connect rect (at -1.23444 1.23444) (size 2.46888 0.09144) (layers F.SilkS) (clearance 0.0254))
  (pad "" connect rect (at -4.43484 1.32588) (size 0.82296 0.09144) (layers F.SilkS) (clearance 0.0254))
  (pad "" connect rect (at -1.23444 1.32588) (size 2.46888 0.09144) (layers F.SilkS) (clearance 0.0254))
  (pad "" connect rect (at -4.52628 1.41732) (size 0.82296 0.09144) (layers F.SilkS) (clearance 0.0254))
  (pad "" connect rect (at -1.23444 1.41732) (size 2.286 0.09144) (layers F.SilkS) (clearance 0.0254))
  (pad "" connect rect (at -4.52628 1.50876) (size 0.64008 0.09144) (layers F.SilkS) (clearance 0.0254))
  (pad "" connect rect (at -1.23444 1.50876) (size 2.286 0.09144) (layers F.SilkS) (clearance 0.0254))
  (pad "" connect rect (at -1.143 1.6002) (size 2.10312 0.09144) (layers F.SilkS) (clearance 0.0254))
  (pad "" connect rect (at -1.55448 1.69164) (size 0.9144 0.09144) (layers F.SilkS) (clearance 0.0254))
  (pad "" connect rect (at -1.50876 1.78308) (size 0.27432 0.09144) (layers F.SilkS) (clearance 0.0254))
  (pad "" connect rect (at -1.55448 1.87452) (size 0.18288 0.09144) (layers F.SilkS) (clearance 0.0254)))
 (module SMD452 (layer F.Cu) (at 163 87 180) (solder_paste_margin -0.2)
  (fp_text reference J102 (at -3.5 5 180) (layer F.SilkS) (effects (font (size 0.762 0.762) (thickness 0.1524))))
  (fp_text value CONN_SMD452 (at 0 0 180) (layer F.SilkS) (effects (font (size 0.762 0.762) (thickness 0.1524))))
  (pad 3 smd rect (at -5.7 -2 180) (size 2.6 2.2) (layers F.Cu F.Paste F.Mask) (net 1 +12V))
  (pad 4 smd rect (at -5.7 2 180) (size 2.6 2.2) (layers F.Cu F.Paste F.Mask) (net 2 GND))
  (pad 1 smd rect (at 5.5 -2 180) (size 3 2.2) (layers F.Cu F.Paste F.Mask) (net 1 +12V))
  (pad 2 smd rect (at 5.5 2 180) (size 3 2.2) (layers F.Cu F.Paste F.Mask) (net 2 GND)))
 (gr_line (start 144 74) (end 170 74) (angle 90) (layer Edge.Cuts) (width 0.15))
 (gr_line (start 144 100) (end 144 74) (angle 90) (layer Edge.Cuts) (width 0.15))
 (gr_line (start 170 100) (end 144 100) (angle 90) (layer Edge.Cuts) (width 0.15))
 (gr_line (start 170 100) (end 170 74) (angle 90) (layer Edge.Cuts) (width 0.15))
 (segment (start 149 84.46) (end 152.46 84.46) (width 3) (layer B.Cu) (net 1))
 (segment (start 152.46 84.46) (end 161 93) (width 3) (layer B.Cu) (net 1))
 (segment (start 157.5 89) (end 157.5 89.5) (width 3) (layer F.Cu) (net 1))
 (segment (start 157.5 89.5) (end 161 93) (width 3) (layer F.Cu) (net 1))
 (segment (start 157.5 89) (end 157.5 93) (width 3) (layer F.Cu) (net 1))
 (segment (start 164.5 89) (end 168 92.5) (width 3) (layer F.Cu) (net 1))
 (segment (start 161 89) (end 161 89.5) (width 3) (layer F.Cu) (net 1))
 (segment (start 161 89.5) (end 164.5 93) (width 3) (layer F.Cu) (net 1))
 (segment (start 164.5 93) (end 164.5 89) (width 3) (layer F.Cu) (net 1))
 (segment (start 161 93) (end 161 89) (width 3) (layer F.Cu) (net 1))
 (segment (start 168 92.5) (end 165 92.5) (width 3) (layer F.Cu) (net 1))
 (segment (start 165 92.5) (end 164.5 93) (width 3) (layer F.Cu) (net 1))
 (segment (start 168.7 89) (end 168.7 91.8) (width 3) (layer F.Cu) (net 1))
 (segment (start 168.7 91.8) (end 168 92.5) (width 3) (layer F.Cu) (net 1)) (via (at 168 92.5) (size 1.5) (layers F.Cu B.Cu) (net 1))
 (segment (start 161 93) (end 164.5 93) (width 3) (layer F.Cu) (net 1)) (via (at 164.5 93) (size 1.5) (layers F.Cu B.Cu) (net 1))
 (segment (start 157.5 93) (end 161 93) (width 3) (layer F.Cu) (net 1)) (via (at 161 93) (size 1.5) (layers F.Cu B.Cu) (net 1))
 (via (at 164.5 89) (size 1.5) (layers F.Cu B.Cu) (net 1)) (via (at 161 89) (size 1.5) (layers F.Cu B.Cu) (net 1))
 (segment (start 157.5 89) (end 161 89) (width 3) (layer F.Cu) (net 1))
 (segment (start 161 89) (end 164.5 89) (width 3) (layer F.Cu) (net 1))
 (segment (start 164.5 89) (end 168.7 89) (width 3) (layer F.Cu) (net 1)) (via (at 157.5 93) (size 1.5) (layers F.Cu B.Cu) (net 1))
 (segment (start 157.5 89) (end 157.5 89) (width 3) (layer F.Cu) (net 1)) (via (at 164.5 81.5) (size 1.5) (layers F.Cu B.Cu) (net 2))
 (segment (start 164.5 85) (end 164.5 81.5) (width 3) (layer F.Cu) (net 2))
 (segment (start 168.7 85) (end 164.5 85) (width 3) (layer F.Cu) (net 2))
 (segment (start 161 85) (end 161 81.5) (width 3) (layer F.Cu) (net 2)) (via (at 161 81.5) (size 1.5) (layers F.Cu B.Cu) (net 2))
 (segment (start 157.5 85) (end 157.5 81.5) (width 3) (layer F.Cu) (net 2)) (via (at 157.5 81.5) (size 1.5) (layers F.Cu B.Cu) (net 2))
 (via (at 161 85) (size 1.5) (layers F.Cu B.Cu) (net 2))
 (segment (start 157.5 85) (end 161 85) (width 3) (layer F.Cu) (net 2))
 (segment (start 161 85) (end 164.5 85) (width 3) (layer F.Cu) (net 2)) (via (at 164.5 85) (size 1.5) (layers F.Cu B.Cu) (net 2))
 (segment (start 157.5 85) (end 153.5 85) (width 3) (layer F.Cu) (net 2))
 (segment (start 151.96 89.54) (end 153.25 88.25) (width 3) (layer F.Cu) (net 2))
 (segment (start 151.96 89.54) (end 149 89.54) (width 3) (layer F.Cu) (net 2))
 (segment (start 153.25 85.25) (end 153.25 88.25) (width 3) (layer F.Cu) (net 2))
 (segment (start 153.5 85) (end 153.25 85.25) (width 3) (layer F.Cu) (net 2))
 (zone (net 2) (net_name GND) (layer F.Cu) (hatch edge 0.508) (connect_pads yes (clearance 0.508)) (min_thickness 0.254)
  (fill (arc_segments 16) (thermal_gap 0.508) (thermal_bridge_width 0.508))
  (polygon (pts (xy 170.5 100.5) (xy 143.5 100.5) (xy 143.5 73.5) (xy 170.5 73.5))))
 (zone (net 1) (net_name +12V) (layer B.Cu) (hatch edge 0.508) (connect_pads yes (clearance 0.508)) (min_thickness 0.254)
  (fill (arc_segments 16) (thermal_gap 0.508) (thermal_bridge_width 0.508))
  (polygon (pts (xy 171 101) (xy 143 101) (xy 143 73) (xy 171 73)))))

